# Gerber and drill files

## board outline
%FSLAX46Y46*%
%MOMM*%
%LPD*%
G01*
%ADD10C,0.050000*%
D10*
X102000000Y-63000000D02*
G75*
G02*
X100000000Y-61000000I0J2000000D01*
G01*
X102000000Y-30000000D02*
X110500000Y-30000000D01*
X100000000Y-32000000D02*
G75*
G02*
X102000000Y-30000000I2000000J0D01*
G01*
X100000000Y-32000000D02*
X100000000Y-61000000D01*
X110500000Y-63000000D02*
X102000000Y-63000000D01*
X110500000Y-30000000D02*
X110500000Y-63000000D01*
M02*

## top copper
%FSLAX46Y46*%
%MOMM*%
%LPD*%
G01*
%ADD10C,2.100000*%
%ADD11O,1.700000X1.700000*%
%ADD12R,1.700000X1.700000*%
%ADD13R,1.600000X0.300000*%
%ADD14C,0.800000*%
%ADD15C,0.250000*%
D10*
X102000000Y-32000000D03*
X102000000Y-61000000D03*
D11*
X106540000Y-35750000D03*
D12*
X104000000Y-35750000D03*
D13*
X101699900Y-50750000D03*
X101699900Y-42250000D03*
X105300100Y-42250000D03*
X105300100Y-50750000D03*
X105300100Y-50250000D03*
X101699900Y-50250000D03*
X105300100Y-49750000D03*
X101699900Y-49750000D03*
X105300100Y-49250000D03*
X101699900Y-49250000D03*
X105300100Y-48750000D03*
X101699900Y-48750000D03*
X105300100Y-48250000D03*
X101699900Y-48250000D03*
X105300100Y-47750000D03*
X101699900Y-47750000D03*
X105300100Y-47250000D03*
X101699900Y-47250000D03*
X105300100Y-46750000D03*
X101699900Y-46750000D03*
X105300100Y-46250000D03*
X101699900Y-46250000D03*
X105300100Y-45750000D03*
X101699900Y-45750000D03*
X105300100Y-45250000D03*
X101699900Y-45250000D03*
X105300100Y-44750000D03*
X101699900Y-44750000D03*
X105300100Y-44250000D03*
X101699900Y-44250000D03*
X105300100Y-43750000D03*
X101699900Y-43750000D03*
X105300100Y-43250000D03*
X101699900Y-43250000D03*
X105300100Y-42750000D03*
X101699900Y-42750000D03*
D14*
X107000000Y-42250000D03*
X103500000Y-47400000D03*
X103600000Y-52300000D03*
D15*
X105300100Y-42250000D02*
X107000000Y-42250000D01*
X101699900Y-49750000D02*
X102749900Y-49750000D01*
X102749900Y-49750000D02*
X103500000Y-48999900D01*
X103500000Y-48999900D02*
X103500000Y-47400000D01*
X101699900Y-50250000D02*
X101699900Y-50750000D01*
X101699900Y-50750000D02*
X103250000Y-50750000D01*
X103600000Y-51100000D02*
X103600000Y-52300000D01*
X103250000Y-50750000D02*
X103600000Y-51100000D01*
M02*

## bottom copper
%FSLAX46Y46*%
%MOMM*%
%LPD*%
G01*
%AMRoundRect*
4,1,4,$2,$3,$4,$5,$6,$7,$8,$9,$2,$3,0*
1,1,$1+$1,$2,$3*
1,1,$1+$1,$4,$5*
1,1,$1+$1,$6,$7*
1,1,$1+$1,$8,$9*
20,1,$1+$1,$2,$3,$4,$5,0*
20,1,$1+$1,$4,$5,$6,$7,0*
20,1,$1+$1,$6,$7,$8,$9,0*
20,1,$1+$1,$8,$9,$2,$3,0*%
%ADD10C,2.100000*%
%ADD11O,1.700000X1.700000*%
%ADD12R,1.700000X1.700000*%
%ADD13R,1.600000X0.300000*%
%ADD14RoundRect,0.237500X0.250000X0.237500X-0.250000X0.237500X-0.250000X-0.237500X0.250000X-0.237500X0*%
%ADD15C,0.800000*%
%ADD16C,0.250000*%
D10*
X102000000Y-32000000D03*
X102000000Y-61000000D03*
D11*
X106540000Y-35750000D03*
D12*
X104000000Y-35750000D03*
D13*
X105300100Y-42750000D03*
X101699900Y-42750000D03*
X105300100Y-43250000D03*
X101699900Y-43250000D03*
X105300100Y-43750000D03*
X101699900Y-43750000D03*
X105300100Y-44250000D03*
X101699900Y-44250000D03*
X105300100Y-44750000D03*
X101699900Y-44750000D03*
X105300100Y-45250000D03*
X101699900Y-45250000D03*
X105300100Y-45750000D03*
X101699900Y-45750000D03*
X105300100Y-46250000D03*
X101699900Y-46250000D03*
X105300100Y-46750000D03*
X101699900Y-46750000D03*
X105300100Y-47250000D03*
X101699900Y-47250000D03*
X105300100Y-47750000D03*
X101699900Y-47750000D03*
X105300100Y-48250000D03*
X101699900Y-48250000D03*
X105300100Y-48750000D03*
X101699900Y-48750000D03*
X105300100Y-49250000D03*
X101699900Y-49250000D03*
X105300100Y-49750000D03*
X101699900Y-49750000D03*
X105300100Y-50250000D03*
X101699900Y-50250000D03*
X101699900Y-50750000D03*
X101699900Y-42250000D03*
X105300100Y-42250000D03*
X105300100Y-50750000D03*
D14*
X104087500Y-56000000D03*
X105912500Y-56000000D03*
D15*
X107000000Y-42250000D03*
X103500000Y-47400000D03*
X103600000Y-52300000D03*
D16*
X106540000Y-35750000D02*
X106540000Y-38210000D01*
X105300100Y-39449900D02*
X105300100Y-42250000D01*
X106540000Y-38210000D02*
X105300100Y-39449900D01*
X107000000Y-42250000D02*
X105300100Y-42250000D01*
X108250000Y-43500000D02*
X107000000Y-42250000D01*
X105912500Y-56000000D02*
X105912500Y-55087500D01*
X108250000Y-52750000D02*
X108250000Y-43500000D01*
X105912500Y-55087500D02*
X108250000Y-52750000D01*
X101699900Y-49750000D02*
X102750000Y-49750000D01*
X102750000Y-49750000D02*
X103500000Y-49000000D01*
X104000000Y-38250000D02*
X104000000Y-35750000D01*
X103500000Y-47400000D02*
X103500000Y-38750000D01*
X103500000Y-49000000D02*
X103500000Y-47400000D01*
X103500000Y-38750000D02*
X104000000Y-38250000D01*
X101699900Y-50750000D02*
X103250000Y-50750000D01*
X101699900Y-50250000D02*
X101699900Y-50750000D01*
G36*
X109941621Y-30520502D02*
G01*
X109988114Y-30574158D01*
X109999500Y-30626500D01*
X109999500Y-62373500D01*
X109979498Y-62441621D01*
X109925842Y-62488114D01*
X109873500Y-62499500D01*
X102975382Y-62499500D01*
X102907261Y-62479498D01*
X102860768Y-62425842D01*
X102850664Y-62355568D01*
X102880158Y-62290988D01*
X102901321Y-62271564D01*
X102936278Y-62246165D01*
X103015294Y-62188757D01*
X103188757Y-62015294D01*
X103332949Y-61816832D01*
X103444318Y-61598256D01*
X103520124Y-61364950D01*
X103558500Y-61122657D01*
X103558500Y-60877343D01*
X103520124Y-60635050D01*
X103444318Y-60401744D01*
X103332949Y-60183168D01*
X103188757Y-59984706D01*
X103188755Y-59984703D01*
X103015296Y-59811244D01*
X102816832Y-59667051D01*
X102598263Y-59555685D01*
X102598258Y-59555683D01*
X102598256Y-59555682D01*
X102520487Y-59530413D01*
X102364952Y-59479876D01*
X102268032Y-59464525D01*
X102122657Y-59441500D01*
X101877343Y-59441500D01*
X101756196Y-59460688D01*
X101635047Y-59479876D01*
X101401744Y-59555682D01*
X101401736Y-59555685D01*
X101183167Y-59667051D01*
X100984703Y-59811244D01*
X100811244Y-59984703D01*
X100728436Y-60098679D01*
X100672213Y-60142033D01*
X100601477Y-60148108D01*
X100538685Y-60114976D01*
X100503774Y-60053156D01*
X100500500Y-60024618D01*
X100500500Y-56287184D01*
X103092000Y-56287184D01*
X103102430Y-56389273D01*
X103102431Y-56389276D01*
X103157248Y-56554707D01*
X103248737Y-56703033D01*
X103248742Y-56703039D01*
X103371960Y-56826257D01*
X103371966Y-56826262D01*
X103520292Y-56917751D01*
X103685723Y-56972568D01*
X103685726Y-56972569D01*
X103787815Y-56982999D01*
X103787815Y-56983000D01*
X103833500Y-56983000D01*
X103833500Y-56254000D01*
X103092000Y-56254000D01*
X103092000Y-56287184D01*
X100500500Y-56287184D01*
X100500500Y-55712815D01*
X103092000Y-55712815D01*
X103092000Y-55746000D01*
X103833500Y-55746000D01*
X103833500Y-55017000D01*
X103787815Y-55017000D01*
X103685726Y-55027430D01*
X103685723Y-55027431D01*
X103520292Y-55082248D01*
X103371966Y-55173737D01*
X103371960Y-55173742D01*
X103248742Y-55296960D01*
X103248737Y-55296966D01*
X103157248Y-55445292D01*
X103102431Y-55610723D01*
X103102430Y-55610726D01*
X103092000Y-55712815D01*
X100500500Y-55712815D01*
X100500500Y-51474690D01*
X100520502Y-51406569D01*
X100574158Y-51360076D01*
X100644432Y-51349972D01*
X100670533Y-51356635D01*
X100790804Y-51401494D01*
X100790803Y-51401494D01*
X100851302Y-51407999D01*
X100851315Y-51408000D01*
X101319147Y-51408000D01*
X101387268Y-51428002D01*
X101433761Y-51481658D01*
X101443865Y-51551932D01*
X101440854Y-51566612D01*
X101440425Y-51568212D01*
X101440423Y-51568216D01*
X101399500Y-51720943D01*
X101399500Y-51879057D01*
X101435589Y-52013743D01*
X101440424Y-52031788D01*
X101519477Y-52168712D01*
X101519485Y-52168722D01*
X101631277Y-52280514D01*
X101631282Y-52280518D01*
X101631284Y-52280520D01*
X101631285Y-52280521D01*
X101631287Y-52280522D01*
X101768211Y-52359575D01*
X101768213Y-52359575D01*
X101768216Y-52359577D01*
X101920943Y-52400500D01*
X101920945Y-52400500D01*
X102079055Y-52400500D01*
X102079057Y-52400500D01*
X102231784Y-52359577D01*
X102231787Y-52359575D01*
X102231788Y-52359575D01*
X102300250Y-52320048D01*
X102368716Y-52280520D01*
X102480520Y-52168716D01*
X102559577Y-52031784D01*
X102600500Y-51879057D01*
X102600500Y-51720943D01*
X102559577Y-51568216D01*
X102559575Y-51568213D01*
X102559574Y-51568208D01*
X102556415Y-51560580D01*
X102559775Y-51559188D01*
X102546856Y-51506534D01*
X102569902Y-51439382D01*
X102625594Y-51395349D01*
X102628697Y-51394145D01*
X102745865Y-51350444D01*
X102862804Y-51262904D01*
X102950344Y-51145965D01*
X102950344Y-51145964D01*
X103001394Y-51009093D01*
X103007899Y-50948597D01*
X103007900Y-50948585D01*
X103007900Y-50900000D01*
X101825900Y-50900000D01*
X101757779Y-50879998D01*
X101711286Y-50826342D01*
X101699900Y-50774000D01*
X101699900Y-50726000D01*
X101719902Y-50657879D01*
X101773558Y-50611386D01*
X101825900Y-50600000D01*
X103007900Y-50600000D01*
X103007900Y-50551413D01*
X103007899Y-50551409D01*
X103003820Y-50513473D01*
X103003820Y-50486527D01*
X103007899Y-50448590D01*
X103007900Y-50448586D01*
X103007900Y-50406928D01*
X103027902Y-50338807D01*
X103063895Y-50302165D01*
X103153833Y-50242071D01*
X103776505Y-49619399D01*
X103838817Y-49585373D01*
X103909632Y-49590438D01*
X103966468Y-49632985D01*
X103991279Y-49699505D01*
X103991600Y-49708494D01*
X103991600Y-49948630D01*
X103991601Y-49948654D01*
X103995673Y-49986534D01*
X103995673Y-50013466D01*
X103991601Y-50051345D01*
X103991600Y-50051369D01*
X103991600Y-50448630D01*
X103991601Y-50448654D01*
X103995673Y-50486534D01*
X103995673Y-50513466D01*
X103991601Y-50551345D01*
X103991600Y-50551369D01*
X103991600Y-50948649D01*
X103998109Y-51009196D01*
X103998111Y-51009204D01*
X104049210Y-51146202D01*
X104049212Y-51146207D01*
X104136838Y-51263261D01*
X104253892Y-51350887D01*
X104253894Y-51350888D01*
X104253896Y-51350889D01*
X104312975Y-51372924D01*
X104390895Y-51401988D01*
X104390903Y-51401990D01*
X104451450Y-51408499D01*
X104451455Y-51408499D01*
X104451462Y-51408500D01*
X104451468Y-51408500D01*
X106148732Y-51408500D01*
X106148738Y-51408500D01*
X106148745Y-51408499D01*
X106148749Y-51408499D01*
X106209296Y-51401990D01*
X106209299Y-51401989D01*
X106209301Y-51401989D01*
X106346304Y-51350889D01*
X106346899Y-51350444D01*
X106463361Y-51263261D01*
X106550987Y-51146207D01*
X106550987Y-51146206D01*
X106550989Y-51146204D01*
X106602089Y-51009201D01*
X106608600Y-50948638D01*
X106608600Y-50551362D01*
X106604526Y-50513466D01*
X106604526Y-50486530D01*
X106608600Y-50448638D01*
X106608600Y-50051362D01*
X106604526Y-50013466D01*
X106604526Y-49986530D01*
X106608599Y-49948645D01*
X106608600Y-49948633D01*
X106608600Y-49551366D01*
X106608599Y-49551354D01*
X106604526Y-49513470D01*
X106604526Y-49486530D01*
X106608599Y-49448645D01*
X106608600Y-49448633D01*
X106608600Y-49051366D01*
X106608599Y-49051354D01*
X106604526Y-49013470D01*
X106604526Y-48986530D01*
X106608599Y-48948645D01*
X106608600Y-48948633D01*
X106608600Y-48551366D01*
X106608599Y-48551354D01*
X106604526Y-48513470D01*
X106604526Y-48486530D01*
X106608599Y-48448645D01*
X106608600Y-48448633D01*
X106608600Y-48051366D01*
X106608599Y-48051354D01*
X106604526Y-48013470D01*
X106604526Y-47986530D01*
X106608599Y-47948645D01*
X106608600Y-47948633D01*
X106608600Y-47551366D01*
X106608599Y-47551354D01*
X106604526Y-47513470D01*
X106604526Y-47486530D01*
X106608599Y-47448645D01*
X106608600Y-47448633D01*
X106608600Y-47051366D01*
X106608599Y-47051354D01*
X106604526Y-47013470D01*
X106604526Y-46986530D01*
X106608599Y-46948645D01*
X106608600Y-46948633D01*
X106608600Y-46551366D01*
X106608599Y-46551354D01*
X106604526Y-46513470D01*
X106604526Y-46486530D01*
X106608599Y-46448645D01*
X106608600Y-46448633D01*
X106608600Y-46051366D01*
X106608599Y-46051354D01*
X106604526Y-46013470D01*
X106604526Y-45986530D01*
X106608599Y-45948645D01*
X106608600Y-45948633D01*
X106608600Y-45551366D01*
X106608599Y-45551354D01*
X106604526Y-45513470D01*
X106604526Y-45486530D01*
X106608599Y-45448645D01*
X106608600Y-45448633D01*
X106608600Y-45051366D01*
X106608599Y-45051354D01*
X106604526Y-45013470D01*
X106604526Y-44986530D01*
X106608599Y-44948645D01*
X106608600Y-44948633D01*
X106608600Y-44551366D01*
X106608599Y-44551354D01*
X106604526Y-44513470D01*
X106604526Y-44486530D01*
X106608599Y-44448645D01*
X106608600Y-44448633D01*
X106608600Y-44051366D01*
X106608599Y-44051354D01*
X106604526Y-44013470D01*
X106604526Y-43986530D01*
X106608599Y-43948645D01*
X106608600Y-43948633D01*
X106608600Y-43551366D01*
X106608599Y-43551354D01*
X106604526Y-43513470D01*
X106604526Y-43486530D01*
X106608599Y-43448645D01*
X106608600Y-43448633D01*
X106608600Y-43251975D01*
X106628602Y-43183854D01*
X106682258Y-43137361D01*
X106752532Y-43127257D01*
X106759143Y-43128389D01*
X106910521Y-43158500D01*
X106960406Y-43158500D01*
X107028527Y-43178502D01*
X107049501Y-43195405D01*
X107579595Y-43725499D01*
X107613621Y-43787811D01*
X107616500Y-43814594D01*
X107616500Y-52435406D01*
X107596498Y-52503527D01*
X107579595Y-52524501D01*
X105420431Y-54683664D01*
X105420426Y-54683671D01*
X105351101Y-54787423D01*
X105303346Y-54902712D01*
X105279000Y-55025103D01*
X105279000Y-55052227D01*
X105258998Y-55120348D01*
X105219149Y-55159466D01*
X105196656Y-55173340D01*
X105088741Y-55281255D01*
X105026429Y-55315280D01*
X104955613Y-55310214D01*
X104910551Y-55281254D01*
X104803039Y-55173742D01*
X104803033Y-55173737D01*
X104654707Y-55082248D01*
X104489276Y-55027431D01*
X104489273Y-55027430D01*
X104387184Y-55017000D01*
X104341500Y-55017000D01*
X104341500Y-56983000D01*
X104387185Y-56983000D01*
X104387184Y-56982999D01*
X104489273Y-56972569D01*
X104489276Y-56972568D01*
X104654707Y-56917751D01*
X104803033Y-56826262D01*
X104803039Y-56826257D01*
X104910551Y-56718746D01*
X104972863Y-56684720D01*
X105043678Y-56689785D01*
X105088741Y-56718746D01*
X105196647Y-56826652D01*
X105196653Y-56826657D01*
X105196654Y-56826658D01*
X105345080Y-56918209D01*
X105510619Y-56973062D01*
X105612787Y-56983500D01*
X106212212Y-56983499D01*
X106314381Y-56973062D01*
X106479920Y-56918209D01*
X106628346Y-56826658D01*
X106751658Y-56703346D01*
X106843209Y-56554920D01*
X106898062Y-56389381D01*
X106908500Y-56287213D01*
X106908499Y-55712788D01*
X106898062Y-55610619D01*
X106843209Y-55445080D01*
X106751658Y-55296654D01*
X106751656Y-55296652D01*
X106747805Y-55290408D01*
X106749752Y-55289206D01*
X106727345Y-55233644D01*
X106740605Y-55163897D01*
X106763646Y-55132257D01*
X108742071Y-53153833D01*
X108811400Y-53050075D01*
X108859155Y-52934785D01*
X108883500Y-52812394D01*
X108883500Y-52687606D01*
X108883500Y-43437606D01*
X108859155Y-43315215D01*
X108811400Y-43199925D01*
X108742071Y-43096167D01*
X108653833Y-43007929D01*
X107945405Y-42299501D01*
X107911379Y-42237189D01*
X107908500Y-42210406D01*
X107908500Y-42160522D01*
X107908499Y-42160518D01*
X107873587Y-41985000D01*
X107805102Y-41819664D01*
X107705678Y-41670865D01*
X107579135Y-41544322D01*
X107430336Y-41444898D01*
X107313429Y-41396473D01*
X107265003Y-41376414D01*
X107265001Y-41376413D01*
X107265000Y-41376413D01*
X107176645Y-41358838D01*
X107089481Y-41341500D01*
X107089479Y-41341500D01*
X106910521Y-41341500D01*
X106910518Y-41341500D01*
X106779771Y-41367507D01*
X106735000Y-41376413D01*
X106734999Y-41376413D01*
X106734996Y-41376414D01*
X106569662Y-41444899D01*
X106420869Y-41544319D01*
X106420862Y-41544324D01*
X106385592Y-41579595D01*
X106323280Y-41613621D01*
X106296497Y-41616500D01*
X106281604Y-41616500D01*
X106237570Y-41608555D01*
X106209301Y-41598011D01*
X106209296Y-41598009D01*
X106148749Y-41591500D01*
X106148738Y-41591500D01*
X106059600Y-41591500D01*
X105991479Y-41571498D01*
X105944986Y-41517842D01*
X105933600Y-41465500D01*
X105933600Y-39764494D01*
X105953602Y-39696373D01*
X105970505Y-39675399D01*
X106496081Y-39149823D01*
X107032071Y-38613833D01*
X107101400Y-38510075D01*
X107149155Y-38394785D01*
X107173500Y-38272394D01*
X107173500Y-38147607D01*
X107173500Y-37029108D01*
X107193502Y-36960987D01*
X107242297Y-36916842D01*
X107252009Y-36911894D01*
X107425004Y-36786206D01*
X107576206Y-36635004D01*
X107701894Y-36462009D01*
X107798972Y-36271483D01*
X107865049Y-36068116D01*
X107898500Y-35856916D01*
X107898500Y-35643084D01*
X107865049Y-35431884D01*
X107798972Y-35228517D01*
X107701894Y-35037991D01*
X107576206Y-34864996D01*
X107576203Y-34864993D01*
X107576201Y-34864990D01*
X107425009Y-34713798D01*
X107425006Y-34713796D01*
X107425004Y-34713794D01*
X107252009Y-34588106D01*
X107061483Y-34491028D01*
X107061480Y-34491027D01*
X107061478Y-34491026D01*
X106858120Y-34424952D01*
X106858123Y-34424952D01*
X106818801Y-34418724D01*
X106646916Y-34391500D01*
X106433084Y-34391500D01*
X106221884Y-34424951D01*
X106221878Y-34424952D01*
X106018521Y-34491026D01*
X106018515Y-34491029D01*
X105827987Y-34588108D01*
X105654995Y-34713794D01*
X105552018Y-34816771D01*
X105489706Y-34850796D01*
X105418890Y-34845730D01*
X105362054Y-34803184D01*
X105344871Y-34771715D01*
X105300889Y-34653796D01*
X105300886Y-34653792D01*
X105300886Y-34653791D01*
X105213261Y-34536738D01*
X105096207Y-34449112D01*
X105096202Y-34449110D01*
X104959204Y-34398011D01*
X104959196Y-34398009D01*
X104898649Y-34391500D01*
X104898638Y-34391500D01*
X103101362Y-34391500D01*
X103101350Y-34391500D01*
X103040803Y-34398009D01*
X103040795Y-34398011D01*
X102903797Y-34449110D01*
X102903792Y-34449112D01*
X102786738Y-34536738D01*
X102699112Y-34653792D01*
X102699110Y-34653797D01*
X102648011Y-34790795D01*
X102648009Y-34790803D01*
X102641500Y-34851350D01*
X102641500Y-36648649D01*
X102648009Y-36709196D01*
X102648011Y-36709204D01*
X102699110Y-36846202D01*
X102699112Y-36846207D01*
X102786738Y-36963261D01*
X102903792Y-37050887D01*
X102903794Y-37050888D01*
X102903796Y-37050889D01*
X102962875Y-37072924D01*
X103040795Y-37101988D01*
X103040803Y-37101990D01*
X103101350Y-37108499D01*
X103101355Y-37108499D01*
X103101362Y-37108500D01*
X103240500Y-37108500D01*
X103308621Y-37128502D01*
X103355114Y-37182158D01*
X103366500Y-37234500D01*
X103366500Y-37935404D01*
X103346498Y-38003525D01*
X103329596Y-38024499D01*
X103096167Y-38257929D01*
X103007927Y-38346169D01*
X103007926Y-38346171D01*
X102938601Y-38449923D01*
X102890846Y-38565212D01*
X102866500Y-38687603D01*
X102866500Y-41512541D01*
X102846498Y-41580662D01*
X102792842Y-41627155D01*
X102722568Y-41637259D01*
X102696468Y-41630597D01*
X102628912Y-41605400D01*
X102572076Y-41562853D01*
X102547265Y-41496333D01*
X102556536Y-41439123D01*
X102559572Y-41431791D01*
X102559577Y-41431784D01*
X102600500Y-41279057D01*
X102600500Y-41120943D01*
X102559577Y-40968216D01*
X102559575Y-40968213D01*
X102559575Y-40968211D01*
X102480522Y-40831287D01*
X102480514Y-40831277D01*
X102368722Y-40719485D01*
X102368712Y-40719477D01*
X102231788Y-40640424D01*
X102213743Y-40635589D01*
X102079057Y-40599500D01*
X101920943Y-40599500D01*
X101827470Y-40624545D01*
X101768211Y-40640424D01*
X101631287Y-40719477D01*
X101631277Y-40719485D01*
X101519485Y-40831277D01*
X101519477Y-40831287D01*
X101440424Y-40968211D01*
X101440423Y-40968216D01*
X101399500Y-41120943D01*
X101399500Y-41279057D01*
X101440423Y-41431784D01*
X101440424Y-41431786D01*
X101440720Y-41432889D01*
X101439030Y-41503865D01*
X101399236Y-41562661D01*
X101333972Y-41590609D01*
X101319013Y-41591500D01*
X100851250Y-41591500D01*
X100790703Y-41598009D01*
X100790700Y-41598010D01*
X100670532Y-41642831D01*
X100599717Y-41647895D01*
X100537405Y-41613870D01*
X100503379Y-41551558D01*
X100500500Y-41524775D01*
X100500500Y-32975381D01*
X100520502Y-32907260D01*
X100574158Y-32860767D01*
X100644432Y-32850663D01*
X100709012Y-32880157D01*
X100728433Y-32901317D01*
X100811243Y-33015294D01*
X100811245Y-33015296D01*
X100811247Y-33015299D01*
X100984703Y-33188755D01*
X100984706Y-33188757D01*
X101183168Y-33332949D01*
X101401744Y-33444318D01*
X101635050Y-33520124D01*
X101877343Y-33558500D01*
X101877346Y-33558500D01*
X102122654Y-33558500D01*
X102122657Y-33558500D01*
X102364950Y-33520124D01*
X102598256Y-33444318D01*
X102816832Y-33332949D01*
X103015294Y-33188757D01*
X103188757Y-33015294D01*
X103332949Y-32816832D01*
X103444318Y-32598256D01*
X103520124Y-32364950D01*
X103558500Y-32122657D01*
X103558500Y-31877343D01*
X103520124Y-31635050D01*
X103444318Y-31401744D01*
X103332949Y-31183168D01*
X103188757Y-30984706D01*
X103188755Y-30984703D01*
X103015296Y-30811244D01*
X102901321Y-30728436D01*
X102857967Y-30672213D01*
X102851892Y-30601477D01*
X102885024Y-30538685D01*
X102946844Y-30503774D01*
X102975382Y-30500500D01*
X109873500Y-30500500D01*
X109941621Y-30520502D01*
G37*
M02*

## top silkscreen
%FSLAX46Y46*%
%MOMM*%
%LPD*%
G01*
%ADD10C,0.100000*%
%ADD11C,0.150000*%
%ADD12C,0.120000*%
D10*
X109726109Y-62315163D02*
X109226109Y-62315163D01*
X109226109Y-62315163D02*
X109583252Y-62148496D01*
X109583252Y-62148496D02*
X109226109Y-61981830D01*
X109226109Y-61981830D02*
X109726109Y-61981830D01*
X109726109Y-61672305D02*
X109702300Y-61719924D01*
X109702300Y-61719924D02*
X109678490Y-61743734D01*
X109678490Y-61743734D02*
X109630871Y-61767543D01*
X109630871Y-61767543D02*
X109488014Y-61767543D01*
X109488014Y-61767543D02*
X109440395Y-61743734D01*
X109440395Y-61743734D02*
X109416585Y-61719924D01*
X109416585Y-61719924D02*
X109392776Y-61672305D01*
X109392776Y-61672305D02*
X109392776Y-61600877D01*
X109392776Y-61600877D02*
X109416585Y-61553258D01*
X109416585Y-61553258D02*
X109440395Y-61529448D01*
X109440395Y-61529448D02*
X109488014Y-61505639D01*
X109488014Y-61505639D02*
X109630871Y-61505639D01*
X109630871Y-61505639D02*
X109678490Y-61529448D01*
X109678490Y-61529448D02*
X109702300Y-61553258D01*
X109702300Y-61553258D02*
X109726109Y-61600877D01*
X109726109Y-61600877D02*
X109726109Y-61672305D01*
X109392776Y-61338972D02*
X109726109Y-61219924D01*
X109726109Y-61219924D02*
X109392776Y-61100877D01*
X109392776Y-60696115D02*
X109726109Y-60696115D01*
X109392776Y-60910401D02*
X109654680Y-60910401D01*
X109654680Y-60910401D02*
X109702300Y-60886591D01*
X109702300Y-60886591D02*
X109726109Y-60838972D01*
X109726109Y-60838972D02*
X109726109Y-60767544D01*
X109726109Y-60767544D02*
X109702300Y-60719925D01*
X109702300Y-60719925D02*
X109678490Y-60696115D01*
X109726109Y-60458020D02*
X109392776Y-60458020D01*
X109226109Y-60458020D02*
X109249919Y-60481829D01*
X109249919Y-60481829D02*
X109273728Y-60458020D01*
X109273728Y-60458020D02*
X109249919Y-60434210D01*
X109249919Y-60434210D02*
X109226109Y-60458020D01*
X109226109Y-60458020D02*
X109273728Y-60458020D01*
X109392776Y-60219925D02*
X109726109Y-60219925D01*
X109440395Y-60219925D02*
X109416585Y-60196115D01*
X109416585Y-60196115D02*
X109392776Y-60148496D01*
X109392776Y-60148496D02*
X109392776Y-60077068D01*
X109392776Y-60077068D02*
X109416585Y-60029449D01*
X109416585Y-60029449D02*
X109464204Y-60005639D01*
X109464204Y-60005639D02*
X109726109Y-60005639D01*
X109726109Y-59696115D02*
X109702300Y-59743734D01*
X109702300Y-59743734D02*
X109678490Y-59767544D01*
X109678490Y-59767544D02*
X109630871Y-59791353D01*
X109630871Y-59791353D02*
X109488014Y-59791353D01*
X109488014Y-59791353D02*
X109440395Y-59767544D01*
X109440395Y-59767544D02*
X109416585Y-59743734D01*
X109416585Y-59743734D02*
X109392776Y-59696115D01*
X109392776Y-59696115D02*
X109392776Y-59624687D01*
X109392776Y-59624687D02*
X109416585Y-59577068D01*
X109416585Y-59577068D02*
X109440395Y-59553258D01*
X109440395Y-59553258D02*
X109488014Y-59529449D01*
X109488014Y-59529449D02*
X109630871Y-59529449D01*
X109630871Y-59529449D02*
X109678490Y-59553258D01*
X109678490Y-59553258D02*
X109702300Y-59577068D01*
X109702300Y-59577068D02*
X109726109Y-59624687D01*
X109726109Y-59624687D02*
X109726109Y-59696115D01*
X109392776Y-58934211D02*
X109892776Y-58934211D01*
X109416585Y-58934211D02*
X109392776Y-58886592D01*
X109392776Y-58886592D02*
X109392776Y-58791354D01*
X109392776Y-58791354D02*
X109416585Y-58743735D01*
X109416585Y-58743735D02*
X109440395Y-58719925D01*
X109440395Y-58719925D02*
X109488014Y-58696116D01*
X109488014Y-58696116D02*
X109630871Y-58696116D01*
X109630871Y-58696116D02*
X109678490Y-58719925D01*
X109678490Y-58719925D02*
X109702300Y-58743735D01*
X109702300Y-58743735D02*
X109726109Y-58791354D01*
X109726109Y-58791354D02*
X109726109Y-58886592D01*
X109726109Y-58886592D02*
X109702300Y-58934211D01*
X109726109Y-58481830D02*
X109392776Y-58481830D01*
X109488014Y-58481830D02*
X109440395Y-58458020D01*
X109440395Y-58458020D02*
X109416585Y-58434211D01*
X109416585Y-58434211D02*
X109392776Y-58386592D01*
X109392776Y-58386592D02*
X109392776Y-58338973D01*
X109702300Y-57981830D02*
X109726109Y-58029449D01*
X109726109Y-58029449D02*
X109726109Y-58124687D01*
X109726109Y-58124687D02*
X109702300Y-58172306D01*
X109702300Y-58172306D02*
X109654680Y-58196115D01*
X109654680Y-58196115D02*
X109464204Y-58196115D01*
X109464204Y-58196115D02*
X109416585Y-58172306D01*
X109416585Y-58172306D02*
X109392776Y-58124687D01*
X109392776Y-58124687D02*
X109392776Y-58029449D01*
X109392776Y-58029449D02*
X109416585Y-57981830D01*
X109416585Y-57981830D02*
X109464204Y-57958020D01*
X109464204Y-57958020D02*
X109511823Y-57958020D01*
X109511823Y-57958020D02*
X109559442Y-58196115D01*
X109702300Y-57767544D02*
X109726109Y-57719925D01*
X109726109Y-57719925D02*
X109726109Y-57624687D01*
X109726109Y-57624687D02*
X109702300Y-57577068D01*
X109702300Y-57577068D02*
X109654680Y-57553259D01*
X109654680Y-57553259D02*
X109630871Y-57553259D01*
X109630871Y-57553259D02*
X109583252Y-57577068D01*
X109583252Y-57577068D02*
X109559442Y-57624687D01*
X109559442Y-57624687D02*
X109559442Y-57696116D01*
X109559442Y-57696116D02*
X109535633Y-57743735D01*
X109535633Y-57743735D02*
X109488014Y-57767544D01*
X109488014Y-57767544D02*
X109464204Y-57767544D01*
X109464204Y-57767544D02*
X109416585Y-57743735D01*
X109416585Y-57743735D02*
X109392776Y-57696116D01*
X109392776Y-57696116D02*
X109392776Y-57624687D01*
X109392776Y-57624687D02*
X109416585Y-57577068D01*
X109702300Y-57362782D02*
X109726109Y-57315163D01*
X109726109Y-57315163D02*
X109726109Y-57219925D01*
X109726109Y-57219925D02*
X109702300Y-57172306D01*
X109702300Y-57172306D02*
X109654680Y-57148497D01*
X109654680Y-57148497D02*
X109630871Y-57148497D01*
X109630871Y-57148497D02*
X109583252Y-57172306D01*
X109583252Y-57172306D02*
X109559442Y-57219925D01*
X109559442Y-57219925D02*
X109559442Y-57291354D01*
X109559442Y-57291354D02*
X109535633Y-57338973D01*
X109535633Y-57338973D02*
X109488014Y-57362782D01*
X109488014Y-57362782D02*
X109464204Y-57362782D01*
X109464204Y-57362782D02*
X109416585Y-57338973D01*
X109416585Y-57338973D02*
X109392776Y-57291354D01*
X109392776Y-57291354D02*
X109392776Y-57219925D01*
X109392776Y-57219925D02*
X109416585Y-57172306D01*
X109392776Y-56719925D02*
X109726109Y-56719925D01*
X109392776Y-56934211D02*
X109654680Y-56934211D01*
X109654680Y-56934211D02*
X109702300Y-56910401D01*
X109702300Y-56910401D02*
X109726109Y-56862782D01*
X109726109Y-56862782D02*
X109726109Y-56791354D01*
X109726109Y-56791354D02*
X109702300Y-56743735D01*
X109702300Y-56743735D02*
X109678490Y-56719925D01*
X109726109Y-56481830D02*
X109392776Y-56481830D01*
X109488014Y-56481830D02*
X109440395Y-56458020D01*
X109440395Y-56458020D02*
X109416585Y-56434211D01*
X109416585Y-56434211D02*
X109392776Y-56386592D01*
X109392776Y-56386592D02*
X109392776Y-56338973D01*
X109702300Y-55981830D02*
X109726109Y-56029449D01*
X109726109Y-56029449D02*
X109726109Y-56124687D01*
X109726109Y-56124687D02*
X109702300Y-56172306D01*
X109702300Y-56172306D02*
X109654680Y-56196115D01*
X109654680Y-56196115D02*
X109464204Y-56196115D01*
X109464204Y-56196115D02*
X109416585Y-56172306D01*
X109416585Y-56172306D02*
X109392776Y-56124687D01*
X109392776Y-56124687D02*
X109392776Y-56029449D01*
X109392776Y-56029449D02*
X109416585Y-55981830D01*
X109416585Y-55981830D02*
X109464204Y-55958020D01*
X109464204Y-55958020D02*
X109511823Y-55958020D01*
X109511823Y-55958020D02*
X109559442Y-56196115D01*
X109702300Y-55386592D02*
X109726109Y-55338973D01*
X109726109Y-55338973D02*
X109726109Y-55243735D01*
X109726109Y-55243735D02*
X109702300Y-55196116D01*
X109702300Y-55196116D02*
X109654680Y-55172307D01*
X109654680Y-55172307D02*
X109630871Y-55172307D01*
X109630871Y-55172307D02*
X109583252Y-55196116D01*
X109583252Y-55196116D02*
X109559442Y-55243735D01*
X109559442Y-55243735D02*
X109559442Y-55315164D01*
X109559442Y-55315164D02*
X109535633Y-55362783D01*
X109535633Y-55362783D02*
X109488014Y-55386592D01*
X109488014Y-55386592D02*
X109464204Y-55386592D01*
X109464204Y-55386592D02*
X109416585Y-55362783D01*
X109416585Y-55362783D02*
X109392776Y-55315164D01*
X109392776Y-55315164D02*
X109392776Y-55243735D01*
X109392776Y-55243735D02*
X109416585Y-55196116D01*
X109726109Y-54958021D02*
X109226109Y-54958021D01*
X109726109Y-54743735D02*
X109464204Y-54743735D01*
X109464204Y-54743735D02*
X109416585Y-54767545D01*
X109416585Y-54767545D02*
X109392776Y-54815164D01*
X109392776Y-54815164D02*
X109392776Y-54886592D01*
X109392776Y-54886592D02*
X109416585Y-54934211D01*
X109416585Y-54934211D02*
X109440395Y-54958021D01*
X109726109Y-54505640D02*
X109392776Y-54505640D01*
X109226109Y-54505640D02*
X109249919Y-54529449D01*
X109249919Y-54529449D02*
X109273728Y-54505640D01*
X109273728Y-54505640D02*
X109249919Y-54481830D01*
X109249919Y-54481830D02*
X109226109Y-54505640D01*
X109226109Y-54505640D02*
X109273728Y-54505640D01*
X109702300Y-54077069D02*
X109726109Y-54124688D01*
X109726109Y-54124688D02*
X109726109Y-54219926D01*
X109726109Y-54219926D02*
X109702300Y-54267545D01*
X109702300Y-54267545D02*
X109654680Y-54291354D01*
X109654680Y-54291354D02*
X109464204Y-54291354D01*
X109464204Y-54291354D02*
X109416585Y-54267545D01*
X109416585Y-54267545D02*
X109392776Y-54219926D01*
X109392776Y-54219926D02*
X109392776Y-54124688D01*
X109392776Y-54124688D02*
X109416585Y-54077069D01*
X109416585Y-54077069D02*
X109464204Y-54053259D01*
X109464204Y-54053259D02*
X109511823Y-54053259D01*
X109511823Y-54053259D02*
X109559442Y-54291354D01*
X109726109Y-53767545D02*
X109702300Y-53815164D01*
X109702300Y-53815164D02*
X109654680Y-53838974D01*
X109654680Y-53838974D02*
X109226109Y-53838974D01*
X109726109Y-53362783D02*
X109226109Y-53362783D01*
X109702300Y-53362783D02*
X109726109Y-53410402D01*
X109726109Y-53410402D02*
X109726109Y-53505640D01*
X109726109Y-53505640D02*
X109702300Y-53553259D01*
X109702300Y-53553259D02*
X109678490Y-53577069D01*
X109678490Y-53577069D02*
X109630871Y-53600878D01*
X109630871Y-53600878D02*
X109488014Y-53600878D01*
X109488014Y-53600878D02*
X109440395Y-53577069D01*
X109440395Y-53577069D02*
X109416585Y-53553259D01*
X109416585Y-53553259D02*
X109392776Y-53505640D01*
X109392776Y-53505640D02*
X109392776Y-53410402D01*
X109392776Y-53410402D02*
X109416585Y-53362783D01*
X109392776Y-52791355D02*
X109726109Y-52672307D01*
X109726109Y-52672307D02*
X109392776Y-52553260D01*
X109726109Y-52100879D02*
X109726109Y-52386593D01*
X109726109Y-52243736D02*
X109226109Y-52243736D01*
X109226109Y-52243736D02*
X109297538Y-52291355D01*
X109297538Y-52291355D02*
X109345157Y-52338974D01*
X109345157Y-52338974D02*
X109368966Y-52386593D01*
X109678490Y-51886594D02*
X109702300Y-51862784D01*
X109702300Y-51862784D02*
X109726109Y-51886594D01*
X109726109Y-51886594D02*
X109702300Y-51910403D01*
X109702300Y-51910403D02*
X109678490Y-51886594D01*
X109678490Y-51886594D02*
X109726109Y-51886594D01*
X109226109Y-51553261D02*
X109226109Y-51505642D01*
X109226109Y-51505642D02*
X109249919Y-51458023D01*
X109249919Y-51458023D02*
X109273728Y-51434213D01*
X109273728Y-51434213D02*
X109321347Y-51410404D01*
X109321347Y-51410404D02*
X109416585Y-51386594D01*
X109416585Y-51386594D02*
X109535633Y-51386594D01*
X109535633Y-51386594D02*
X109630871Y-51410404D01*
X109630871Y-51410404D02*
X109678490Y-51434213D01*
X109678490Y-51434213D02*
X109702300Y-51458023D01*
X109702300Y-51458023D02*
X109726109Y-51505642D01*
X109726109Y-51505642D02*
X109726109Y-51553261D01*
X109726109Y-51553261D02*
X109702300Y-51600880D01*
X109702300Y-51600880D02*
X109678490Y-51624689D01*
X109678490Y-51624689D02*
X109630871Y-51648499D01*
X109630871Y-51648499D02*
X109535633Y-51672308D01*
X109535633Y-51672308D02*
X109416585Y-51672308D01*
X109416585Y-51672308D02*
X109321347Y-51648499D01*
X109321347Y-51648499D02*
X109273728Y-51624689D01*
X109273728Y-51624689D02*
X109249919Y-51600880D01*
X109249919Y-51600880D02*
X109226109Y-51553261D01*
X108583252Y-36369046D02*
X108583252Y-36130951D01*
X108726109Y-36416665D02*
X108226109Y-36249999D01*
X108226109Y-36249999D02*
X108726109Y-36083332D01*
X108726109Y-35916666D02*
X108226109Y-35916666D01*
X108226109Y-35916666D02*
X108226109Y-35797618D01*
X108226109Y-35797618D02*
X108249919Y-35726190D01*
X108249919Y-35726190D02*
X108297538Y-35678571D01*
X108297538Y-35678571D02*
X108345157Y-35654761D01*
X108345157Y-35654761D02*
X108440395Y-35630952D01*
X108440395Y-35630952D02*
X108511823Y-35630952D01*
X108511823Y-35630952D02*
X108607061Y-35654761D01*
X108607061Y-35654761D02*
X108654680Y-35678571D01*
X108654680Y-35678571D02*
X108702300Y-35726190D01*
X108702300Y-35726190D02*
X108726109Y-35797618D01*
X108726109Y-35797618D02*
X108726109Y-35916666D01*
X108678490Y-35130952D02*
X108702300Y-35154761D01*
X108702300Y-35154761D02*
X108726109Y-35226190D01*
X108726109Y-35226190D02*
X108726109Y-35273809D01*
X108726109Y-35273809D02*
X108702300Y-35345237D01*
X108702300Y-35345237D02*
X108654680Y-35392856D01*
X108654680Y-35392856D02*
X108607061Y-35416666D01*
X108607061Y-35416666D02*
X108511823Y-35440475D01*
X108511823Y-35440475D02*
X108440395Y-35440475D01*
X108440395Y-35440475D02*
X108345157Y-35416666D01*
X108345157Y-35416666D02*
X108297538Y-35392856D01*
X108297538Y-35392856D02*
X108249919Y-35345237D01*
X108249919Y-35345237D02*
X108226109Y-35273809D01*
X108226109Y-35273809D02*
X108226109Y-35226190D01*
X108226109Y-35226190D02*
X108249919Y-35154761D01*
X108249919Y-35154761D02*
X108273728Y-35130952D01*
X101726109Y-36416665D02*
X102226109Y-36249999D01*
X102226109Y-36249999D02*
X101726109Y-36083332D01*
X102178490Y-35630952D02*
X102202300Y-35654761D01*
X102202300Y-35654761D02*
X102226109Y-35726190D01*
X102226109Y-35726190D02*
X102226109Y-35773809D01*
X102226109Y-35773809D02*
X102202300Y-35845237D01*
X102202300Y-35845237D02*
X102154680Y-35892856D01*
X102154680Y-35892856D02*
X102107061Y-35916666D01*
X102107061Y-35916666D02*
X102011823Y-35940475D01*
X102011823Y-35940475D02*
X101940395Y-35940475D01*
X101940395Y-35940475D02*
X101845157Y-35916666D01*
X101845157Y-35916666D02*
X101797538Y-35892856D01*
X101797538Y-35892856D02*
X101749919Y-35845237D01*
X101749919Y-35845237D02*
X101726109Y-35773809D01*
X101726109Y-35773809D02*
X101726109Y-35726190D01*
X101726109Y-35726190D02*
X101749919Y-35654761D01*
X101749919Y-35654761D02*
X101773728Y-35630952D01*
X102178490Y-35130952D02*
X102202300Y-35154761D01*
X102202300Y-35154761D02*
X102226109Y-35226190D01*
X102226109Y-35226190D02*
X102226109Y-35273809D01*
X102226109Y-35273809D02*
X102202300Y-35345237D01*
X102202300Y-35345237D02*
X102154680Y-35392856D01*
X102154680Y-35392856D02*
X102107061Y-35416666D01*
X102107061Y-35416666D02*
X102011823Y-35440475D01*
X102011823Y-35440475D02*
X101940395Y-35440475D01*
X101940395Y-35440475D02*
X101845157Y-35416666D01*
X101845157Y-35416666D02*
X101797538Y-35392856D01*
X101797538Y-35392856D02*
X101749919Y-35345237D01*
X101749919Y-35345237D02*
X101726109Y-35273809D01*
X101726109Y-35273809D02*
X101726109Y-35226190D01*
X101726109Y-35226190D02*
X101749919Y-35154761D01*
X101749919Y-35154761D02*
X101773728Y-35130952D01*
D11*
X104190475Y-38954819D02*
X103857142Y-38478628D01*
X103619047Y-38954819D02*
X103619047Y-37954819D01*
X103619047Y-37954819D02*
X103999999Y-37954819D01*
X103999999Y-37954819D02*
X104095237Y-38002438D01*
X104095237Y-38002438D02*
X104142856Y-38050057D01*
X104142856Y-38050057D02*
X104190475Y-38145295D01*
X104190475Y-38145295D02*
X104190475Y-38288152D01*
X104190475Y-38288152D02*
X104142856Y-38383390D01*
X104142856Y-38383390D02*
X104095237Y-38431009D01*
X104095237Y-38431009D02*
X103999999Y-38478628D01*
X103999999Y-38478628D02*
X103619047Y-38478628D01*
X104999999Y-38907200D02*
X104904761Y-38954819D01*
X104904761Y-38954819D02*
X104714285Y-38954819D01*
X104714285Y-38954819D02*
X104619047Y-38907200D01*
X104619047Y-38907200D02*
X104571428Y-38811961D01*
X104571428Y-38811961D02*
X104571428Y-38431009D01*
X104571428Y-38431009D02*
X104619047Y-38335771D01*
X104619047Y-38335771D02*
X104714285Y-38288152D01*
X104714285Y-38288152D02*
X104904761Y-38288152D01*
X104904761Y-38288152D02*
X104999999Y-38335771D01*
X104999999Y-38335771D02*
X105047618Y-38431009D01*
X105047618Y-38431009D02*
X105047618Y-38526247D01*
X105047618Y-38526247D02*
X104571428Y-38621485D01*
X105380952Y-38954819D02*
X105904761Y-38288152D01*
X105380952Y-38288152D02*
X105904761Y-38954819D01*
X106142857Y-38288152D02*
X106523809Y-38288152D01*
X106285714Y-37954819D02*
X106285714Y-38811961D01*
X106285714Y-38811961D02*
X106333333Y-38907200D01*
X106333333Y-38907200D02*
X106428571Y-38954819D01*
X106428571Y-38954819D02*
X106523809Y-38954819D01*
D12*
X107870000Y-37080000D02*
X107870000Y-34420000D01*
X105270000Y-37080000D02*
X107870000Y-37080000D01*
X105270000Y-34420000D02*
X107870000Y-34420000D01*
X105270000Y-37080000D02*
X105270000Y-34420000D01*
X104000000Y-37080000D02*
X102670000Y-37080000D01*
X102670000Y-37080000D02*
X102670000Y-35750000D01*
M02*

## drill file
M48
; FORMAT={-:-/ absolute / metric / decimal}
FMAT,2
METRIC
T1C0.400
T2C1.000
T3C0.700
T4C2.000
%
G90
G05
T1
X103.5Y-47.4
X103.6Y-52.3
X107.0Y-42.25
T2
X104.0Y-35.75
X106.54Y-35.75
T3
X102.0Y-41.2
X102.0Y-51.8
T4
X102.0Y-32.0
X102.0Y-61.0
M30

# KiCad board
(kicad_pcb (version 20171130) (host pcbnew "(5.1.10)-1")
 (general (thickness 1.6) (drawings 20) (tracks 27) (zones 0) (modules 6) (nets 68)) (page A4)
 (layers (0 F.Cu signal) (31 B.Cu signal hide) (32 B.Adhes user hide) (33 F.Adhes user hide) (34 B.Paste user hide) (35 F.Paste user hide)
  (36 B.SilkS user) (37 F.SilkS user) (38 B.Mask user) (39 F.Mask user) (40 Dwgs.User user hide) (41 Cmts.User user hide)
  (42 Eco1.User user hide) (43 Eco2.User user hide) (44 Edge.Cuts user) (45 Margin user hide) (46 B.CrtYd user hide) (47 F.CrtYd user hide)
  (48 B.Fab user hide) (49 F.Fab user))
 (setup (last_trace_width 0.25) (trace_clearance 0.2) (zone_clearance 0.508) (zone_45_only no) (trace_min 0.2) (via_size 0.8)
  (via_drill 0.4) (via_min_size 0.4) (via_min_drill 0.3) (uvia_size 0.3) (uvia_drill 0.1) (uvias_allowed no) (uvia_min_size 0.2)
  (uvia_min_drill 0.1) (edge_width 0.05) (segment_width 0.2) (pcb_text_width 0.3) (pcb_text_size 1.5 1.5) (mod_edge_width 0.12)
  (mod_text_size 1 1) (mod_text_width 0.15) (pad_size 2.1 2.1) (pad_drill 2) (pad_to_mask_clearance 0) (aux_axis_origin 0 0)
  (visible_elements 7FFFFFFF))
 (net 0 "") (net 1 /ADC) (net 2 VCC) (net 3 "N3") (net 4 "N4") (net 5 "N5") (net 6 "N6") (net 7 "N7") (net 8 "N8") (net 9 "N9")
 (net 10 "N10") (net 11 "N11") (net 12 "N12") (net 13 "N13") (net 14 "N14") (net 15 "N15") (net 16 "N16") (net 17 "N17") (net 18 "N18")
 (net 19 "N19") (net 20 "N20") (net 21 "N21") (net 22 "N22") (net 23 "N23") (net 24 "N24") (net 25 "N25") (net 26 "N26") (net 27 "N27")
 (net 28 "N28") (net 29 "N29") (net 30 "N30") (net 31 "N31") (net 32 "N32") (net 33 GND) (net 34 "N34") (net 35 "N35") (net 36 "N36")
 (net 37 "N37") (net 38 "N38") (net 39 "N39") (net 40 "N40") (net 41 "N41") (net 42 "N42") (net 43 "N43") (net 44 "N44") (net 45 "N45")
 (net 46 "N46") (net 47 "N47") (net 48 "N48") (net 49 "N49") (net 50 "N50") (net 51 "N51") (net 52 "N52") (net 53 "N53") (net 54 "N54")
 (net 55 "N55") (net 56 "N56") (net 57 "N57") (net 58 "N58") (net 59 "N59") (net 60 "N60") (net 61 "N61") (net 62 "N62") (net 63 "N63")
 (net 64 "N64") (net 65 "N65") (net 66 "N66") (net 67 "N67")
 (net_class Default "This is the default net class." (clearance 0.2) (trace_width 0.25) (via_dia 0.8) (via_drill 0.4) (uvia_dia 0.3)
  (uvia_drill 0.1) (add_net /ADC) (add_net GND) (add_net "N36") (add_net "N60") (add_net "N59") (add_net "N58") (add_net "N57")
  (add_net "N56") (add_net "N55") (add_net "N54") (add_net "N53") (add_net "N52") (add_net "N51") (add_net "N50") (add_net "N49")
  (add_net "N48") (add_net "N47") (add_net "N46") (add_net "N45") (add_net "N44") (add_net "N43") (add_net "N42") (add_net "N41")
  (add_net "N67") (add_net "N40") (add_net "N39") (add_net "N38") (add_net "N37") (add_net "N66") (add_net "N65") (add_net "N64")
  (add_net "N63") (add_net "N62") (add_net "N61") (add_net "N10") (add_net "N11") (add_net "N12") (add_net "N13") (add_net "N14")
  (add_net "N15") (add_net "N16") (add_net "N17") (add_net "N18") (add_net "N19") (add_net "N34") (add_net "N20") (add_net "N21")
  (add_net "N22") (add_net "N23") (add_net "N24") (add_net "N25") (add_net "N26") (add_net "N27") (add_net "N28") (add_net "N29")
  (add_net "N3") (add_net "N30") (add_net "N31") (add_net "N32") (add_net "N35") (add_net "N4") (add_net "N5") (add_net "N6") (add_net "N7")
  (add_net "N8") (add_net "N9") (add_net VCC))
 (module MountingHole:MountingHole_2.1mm (layer F.Cu) (at 102 32)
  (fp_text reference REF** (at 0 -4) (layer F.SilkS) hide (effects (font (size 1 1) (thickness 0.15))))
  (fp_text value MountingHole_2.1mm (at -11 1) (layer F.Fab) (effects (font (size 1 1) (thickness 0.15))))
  (pad "" np_thru_hole circle (at 0 0) (size 2.1 2.1) (drill 2) (layers *.Cu B.Mask)))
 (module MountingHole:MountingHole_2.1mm (layer F.Cu) (at 102 61)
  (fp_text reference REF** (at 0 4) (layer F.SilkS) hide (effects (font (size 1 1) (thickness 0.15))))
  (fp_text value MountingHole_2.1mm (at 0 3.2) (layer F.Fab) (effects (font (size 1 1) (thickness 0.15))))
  (pad "" np_thru_hole circle (at 0 0) (size 2.1 2.1) (drill 2) (layers *.Cu *.Mask)))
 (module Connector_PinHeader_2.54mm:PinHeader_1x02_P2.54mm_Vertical (layer F.Cu) (at 104 35.75 90)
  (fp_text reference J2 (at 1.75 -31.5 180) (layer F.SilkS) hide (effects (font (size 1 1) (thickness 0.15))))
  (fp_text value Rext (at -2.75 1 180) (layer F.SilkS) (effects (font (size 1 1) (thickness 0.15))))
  (fp_line (start -1.33 3.87) (end 1.33 3.87) (layer F.SilkS) (width 0.12))
  (fp_line (start -1.33 1.27) (end -1.33 3.87) (layer F.SilkS) (width 0.12))
  (fp_line (start 1.33 1.27) (end 1.33 3.87) (layer F.SilkS) (width 0.12))
  (fp_line (start -1.33 1.27) (end 1.33 1.27) (layer F.SilkS) (width 0.12))
  (fp_line (start -1.33 0) (end -1.33 -1.33) (layer F.SilkS) (width 0.12))
  (fp_line (start -1.33 -1.33) (end 0 -1.33) (layer F.SilkS) (width 0.12))
  (pad 2 thru_hole oval (at 0 2.54 90) (size 1.7 1.7) (drill 1) (layers *.Cu *.Mask) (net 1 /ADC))
  (pad 1 thru_hole rect (at 0 0 90) (size 1.7 1.7) (drill 1) (layers *.Cu *.Mask) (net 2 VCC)))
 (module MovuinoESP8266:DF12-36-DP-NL (layer B.Cu) (at 103.5 46.5 270)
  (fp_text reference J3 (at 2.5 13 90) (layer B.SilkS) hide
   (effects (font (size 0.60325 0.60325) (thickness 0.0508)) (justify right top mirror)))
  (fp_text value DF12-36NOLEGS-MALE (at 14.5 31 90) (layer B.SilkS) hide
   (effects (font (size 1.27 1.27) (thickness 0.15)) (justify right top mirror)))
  (pad 3 smd rect (at -3.75 -1.8001 270) (size 0.3 1.6) (layers B.Cu B.Mask) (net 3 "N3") (solder_mask_margin 0.1016))
  (pad 4 smd rect (at -3.75 1.8001 270) (size 0.3 1.6) (layers B.Cu B.Mask) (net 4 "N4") (solder_mask_margin 0.1016))
  (pad 5 smd rect (at -3.25 -1.8001 270) (size 0.3 1.6) (layers B.Cu B.Mask) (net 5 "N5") (solder_mask_margin 0.1016))
  (pad 6 smd rect (at -3.25 1.8001 270) (size 0.3 1.6) (layers B.Cu B.Mask) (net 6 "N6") (solder_mask_margin 0.1016))
  (pad 7 smd rect (at -2.75 -1.8001 270) (size 0.3 1.6) (layers B.Cu B.Mask) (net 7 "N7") (solder_mask_margin 0.1016))
  (pad 8 smd rect (at -2.75 1.8001 270) (size 0.3 1.6) (layers B.Cu B.Mask) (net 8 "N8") (solder_mask_margin 0.1016))
  (pad 9 smd rect (at -2.25 -1.8001 270) (size 0.3 1.6) (layers B.Cu B.Mask) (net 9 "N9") (solder_mask_margin 0.1016))
  (pad 10 smd rect (at -2.25 1.8001 270) (size 0.3 1.6) (layers B.Cu B.Mask) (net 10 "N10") (solder_mask_margin 0.1016))
  (pad 11 smd rect (at -1.75 -1.8001 270) (size 0.3 1.6) (layers B.Cu B.Mask) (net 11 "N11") (solder_mask_margin 0.1016))
  (pad 12 smd rect (at -1.75 1.8001 270) (size 0.3 1.6) (layers B.Cu B.Mask) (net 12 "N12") (solder_mask_margin 0.1016))
  (pad 13 smd rect (at -1.25 -1.8001 270) (size 0.3 1.6) (layers B.Cu B.Mask) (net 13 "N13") (solder_mask_margin 0.1016))
  (pad 14 smd rect (at -1.25 1.8001 270) (size 0.3 1.6) (layers B.Cu B.Mask) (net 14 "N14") (solder_mask_margin 0.1016))
  (pad 15 smd rect (at -0.75 -1.8001 270) (size 0.3 1.6) (layers B.Cu B.Mask) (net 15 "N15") (solder_mask_margin 0.1016))
  (pad 16 smd rect (at -0.75 1.8001 270) (size 0.3 1.6) (layers B.Cu B.Mask) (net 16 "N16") (solder_mask_margin 0.1016))
  (pad 17 smd rect (at -0.25 -1.8001 270) (size 0.3 1.6) (layers B.Cu B.Mask) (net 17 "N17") (solder_mask_margin 0.1016))
  (pad 18 smd rect (at -0.25 1.8001 270) (size 0.3 1.6) (layers B.Cu B.Mask) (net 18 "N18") (solder_mask_margin 0.1016))
  (pad 19 smd rect (at 0.25 -1.8001 270) (size 0.3 1.6) (layers B.Cu B.Mask) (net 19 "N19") (solder_mask_margin 0.1016))
  (pad 20 smd rect (at 0.25 1.8001 270) (size 0.3 1.6) (layers B.Cu B.Mask) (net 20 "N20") (solder_mask_margin 0.1016))
  (pad 21 smd rect (at 0.75 -1.8001 270) (size 0.3 1.6) (layers B.Cu B.Mask) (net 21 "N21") (solder_mask_margin 0.1016))
  (pad 22 smd rect (at 0.75 1.8001 270) (size 0.3 1.6) (layers B.Cu B.Mask) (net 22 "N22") (solder_mask_margin 0.1016))
  (pad 23 smd rect (at 1.25 -1.8001 270) (size 0.3 1.6) (layers B.Cu B.Mask) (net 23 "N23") (solder_mask_margin 0.1016))
  (pad 24 smd rect (at 1.25 1.8001 270) (size 0.3 1.6) (layers B.Cu B.Mask) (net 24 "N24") (solder_mask_margin 0.1016))
  (pad 25 smd rect (at 1.75 -1.8001 270) (size 0.3 1.6) (layers B.Cu B.Mask) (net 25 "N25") (solder_mask_margin 0.1016))
  (pad 26 smd rect (at 1.75 1.8001 270) (size 0.3 1.6) (layers B.Cu B.Mask) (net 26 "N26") (solder_mask_margin 0.1016))
  (pad 27 smd rect (at 2.25 -1.8001 270) (size 0.3 1.6) (layers B.Cu B.Mask) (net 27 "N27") (solder_mask_margin 0.1016))
  (pad 28 smd rect (at 2.25 1.8001 270) (size 0.3 1.6) (layers B.Cu B.Mask) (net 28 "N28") (solder_mask_margin 0.1016))
  (pad 29 smd rect (at 2.75 -1.8001 270) (size 0.3 1.6) (layers B.Cu B.Mask) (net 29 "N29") (solder_mask_margin 0.1016))
  (pad 30 smd rect (at 2.75 1.8001 270) (size 0.3 1.6) (layers B.Cu B.Mask) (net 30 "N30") (solder_mask_margin 0.1016))
  (pad 31 smd rect (at 3.25 -1.8001 270) (size 0.3 1.6) (layers B.Cu B.Mask) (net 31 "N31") (solder_mask_margin 0.1016))
  (pad 32 smd rect (at 3.25 1.8001 270) (size 0.3 1.6) (layers B.Cu B.Mask) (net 2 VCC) (solder_mask_margin 0.1016))
  (pad 33 smd rect (at 3.75 -1.8001 270) (size 0.3 1.6) (layers B.Cu B.Mask) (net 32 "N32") (solder_mask_margin 0.1016))
  (pad 34 smd rect (at 3.75 1.8001 270) (size 0.3 1.6) (layers B.Cu B.Mask) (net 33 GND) (solder_mask_margin 0.1016))
  (pad 36 smd rect (at 4.25 1.8001 270) (size 0.3 1.6) (layers B.Cu B.Mask) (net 33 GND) (solder_mask_margin 0.1016))
  (pad 2 smd rect (at -4.25 1.8001 270) (size 0.3 1.6) (layers B.Cu B.Mask) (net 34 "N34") (solder_mask_margin 0.1016))
  (pad 1 smd rect (at -4.25 -1.8001 270) (size 0.3 1.6) (layers B.Cu B.Mask) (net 1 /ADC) (solder_mask_margin 0.1016))
  (pad 35 smd rect (at 4.25 -1.8001 270) (size 0.3 1.6) (layers B.Cu B.Mask) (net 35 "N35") (solder_mask_margin 0.1016))
  (pad "" np_thru_hole circle (at -5.3 1.5 270) (size 0.7 0.7) (drill 0.7) (layers *.Cu *.Mask))
  (pad "" np_thru_hole circle (at 5.3 1.5 270) (size 0.7 0.7) (drill 0.7) (layers *.Cu *.Mask)))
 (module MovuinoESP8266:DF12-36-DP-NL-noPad (layer F.Cu) (at 103.5 46.5 270)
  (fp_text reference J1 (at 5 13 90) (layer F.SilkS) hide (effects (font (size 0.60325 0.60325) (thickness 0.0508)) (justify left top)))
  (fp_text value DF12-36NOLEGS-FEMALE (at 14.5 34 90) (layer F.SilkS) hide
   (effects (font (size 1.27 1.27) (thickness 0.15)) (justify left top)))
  (pad 35 smd rect (at 4.25 1.8001 270) (size 0.3 1.6) (layers F.Cu F.Mask) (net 33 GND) (solder_mask_margin 0.1016))
  (pad 1 smd rect (at -4.25 1.8001 270) (size 0.3 1.6) (layers F.Cu F.Mask) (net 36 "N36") (solder_mask_margin 0.1016))
  (pad 2 smd rect (at -4.25 -1.8001 270) (size 0.3 1.6) (layers F.Cu F.Mask) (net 1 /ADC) (solder_mask_margin 0.1016))
  (pad 36 smd rect (at 4.25 -1.8001 270) (size 0.3 1.6) (layers F.Cu F.Mask) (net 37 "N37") (solder_mask_margin 0.1016))
  (pad 34 smd rect (at 3.75 -1.8001 270) (size 0.3 1.6) (layers F.Cu F.Mask) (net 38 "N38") (solder_mask_margin 0.1016))
  (pad 33 smd rect (at 3.75 1.8001 270) (size 0.3 1.6) (layers F.Cu F.Mask) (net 33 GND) (solder_mask_margin 0.1016))
  (pad 32 smd rect (at 3.25 -1.8001 270) (size 0.3 1.6) (layers F.Cu F.Mask) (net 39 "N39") (solder_mask_margin 0.1016))
  (pad 31 smd rect (at 3.25 1.8001 270) (size 0.3 1.6) (layers F.Cu F.Mask) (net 2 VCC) (solder_mask_margin 0.1016))
  (pad 30 smd rect (at 2.75 -1.8001 270) (size 0.3 1.6) (layers F.Cu F.Mask) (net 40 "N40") (solder_mask_margin 0.1016))
  (pad 29 smd rect (at 2.75 1.8001 270) (size 0.3 1.6) (layers F.Cu F.Mask) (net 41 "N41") (solder_mask_margin 0.1016))
  (pad 28 smd rect (at 2.25 -1.8001 270) (size 0.3 1.6) (layers F.Cu F.Mask) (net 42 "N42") (solder_mask_margin 0.1016))
  (pad 27 smd rect (at 2.25 1.8001 270) (size 0.3 1.6) (layers F.Cu F.Mask) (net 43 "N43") (solder_mask_margin 0.1016))
  (pad 26 smd rect (at 1.75 -1.8001 270) (size 0.3 1.6) (layers F.Cu F.Mask) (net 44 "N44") (solder_mask_margin 0.1016))
  (pad 25 smd rect (at 1.75 1.8001 270) (size 0.3 1.6) (layers F.Cu F.Mask) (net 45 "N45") (solder_mask_margin 0.1016))
  (pad 24 smd rect (at 1.25 -1.8001 270) (size 0.3 1.6) (layers F.Cu F.Mask) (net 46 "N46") (solder_mask_margin 0.1016))
  (pad 23 smd rect (at 1.25 1.8001 270) (size 0.3 1.6) (layers F.Cu F.Mask) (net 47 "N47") (solder_mask_margin 0.1016))
  (pad 22 smd rect (at 0.75 -1.8001 270) (size 0.3 1.6) (layers F.Cu F.Mask) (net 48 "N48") (solder_mask_margin 0.1016))
  (pad 21 smd rect (at 0.75 1.8001 270) (size 0.3 1.6) (layers F.Cu F.Mask) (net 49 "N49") (solder_mask_margin 0.1016))
  (pad 20 smd rect (at 0.25 -1.8001 270) (size 0.3 1.6) (layers F.Cu F.Mask) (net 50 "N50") (solder_mask_margin 0.1016))
  (pad 19 smd rect (at 0.25 1.8001 270) (size 0.3 1.6) (layers F.Cu F.Mask) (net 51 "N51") (solder_mask_margin 0.1016))
  (pad 18 smd rect (at -0.25 -1.8001 270) (size 0.3 1.6) (layers F.Cu F.Mask) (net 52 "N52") (solder_mask_margin 0.1016))
  (pad 17 smd rect (at -0.25 1.8001 270) (size 0.3 1.6) (layers F.Cu F.Mask) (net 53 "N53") (solder_mask_margin 0.1016))
  (pad 16 smd rect (at -0.75 -1.8001 270) (size 0.3 1.6) (layers F.Cu F.Mask) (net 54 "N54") (solder_mask_margin 0.1016))
  (pad 15 smd rect (at -0.75 1.8001 270) (size 0.3 1.6) (layers F.Cu F.Mask) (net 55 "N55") (solder_mask_margin 0.1016))
  (pad 14 smd rect (at -1.25 -1.8001 270) (size 0.3 1.6) (layers F.Cu F.Mask) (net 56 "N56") (solder_mask_margin 0.1016))
  (pad 13 smd rect (at -1.25 1.8001 270) (size 0.3 1.6) (layers F.Cu F.Mask) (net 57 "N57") (solder_mask_margin 0.1016))
  (pad 12 smd rect (at -1.75 -1.8001 270) (size 0.3 1.6) (layers F.Cu F.Mask) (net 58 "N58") (solder_mask_margin 0.1016))
  (pad 11 smd rect (at -1.75 1.8001 270) (size 0.3 1.6) (layers F.Cu F.Mask) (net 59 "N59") (solder_mask_margin 0.1016))
  (pad 10 smd rect (at -2.25 -1.8001 270) (size 0.3 1.6) (layers F.Cu F.Mask) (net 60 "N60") (solder_mask_margin 0.1016))
  (pad 9 smd rect (at -2.25 1.8001 270) (size 0.3 1.6) (layers F.Cu F.Mask) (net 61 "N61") (solder_mask_margin 0.1016))
  (pad 8 smd rect (at -2.75 -1.8001 270) (size 0.3 1.6) (layers F.Cu F.Mask) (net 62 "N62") (solder_mask_margin 0.1016))
  (pad 7 smd rect (at -2.75 1.8001 270) (size 0.3 1.6) (layers F.Cu F.Mask) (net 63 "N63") (solder_mask_margin 0.1016))
  (pad 6 smd rect (at -3.25 -1.8001 270) (size 0.3 1.6) (layers F.Cu F.Mask) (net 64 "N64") (solder_mask_margin 0.1016))
  (pad 5 smd rect (at -3.25 1.8001 270) (size 0.3 1.6) (layers F.Cu F.Mask) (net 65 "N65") (solder_mask_margin 0.1016))
  (pad 4 smd rect (at -3.75 -1.8001 270) (size 0.3 1.6) (layers F.Cu F.Mask) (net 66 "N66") (solder_mask_margin 0.1016))
  (pad 3 smd rect (at -3.75 1.8001 270) (size 0.3 1.6) (layers F.Cu F.Mask) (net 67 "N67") (solder_mask_margin 0.1016)))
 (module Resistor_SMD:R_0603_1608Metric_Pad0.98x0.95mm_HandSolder (layer B.Cu) (at 105 56 180)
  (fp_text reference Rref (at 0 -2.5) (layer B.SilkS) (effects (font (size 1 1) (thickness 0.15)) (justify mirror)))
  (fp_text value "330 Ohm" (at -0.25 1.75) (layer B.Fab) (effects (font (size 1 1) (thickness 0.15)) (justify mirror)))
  (pad 2 smd roundrect (at 0.9125 0 180) (size 0.975 0.95) (layers B.Cu B.Paste B.Mask) (roundrect_rratio 0.25) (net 33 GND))
  (pad 1 smd roundrect (at -0.9125 0 180) (size 0.975 0.95) (layers B.Cu B.Paste B.Mask) (roundrect_rratio 0.25) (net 1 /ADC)))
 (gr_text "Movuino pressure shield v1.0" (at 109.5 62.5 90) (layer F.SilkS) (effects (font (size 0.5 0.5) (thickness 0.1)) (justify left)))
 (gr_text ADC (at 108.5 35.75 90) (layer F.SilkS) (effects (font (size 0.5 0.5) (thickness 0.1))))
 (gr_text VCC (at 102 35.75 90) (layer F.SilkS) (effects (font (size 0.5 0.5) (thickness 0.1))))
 (gr_arc (start 102 61) (end 100 61) (angle -90) (layer Edge.Cuts) (width 0.05))
 (gr_line (start 102 30) (end 110.5 30) (layer Edge.Cuts) (width 0.05))
 (gr_arc (start 102 32) (end 102 30) (angle -90) (layer Edge.Cuts) (width 0.05))
 (gr_line (start 100 32) (end 100 61) (layer Edge.Cuts) (width 0.05))
 (gr_line (start 110.5 63) (end 102 63) (layer Edge.Cuts) (width 0.05))
 (gr_line (start 110.5 30) (end 110.5 63) (layer Edge.Cuts) (width 0.05))
 (segment (start 106.54 35.75) (end 106.54 38.21) (width 0.25) (layer B.Cu) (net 1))
 (segment (start 105.3001 39.4499) (end 105.3001 42.25) (width 0.25) (layer B.Cu) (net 1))
 (segment (start 106.54 38.21) (end 105.3001 39.4499) (width 0.25) (layer B.Cu) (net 1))
 (segment (start 107 42.25) (end 105.3001 42.25) (width 0.25) (layer B.Cu) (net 1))
 (segment (start 108.25 43.5) (end 107 42.25) (width 0.25) (layer B.Cu) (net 1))
 (segment (start 105.9125 56) (end 105.9125 55.0875) (width 0.25) (layer B.Cu) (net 1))
 (segment (start 108.25 52.75) (end 108.25 43.5) (width 0.25) (layer B.Cu) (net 1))
 (segment (start 105.9125 55.0875) (end 108.25 52.75) (width 0.25) (layer B.Cu) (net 1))
 (via (at 107 42.25) (size 0.8) (drill 0.4) (layers F.Cu B.Cu) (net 1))
 (segment (start 105.3001 42.25) (end 107 42.25) (width 0.25) (layer F.Cu) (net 1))
 (segment (start 101.6999 49.75) (end 102.75 49.75) (width 0.25) (layer B.Cu) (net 2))
 (segment (start 102.75 49.75) (end 103.5 49) (width 0.25) (layer B.Cu) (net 2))
 (segment (start 104 38.25) (end 104 35.75) (width 0.25) (layer B.Cu) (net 2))
 (segment (start 103.5 47.4) (end 103.5 38.75) (width 0.25) (layer B.Cu) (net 2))
 (segment (start 101.6999 49.75) (end 102.7499 49.75) (width 0.25) (layer F.Cu) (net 2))
 (segment (start 102.7499 49.75) (end 103.5 48.9999) (width 0.25) (layer F.Cu) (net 2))
 (segment (start 103.5 48.9999) (end 103.5 47.4) (width 0.25) (layer F.Cu) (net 2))
 (via (at 103.5 47.4) (size 0.8) (drill 0.4) (layers F.Cu B.Cu) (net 2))
 (segment (start 103.5 49) (end 103.5 47.4) (width 0.25) (layer B.Cu) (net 2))
 (segment (start 103.5 38.75) (end 104 38.25) (width 0.25) (layer B.Cu) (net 2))
 (segment (start 101.6999 50.75) (end 103.25 50.75) (width 0.25) (layer B.Cu) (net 33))
 (segment (start 101.6999 50.25) (end 101.6999 50.75) (width 0.25) (layer B.Cu) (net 33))
 (segment (start 101.6999 50.25) (end 101.6999 50.75) (width 0.25) (layer F.Cu) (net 33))
 (segment (start 101.6999 50.75) (end 103.25 50.75) (width 0.25) (layer F.Cu) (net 33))
 (via (at 103.6 52.3) (size 0.8) (drill 0.4) (layers F.Cu B.Cu) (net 33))
 (segment (start 103.6 51.1) (end 103.6 52.3) (width 0.25) (layer F.Cu) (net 33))
 (segment (start 103.25 50.75) (end 103.6 51.1) (width 0.25) (layer F.Cu) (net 33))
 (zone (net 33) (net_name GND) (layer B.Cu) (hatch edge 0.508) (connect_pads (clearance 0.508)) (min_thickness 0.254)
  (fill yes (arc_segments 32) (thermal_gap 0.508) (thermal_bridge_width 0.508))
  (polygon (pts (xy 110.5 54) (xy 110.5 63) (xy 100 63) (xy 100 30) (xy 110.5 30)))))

